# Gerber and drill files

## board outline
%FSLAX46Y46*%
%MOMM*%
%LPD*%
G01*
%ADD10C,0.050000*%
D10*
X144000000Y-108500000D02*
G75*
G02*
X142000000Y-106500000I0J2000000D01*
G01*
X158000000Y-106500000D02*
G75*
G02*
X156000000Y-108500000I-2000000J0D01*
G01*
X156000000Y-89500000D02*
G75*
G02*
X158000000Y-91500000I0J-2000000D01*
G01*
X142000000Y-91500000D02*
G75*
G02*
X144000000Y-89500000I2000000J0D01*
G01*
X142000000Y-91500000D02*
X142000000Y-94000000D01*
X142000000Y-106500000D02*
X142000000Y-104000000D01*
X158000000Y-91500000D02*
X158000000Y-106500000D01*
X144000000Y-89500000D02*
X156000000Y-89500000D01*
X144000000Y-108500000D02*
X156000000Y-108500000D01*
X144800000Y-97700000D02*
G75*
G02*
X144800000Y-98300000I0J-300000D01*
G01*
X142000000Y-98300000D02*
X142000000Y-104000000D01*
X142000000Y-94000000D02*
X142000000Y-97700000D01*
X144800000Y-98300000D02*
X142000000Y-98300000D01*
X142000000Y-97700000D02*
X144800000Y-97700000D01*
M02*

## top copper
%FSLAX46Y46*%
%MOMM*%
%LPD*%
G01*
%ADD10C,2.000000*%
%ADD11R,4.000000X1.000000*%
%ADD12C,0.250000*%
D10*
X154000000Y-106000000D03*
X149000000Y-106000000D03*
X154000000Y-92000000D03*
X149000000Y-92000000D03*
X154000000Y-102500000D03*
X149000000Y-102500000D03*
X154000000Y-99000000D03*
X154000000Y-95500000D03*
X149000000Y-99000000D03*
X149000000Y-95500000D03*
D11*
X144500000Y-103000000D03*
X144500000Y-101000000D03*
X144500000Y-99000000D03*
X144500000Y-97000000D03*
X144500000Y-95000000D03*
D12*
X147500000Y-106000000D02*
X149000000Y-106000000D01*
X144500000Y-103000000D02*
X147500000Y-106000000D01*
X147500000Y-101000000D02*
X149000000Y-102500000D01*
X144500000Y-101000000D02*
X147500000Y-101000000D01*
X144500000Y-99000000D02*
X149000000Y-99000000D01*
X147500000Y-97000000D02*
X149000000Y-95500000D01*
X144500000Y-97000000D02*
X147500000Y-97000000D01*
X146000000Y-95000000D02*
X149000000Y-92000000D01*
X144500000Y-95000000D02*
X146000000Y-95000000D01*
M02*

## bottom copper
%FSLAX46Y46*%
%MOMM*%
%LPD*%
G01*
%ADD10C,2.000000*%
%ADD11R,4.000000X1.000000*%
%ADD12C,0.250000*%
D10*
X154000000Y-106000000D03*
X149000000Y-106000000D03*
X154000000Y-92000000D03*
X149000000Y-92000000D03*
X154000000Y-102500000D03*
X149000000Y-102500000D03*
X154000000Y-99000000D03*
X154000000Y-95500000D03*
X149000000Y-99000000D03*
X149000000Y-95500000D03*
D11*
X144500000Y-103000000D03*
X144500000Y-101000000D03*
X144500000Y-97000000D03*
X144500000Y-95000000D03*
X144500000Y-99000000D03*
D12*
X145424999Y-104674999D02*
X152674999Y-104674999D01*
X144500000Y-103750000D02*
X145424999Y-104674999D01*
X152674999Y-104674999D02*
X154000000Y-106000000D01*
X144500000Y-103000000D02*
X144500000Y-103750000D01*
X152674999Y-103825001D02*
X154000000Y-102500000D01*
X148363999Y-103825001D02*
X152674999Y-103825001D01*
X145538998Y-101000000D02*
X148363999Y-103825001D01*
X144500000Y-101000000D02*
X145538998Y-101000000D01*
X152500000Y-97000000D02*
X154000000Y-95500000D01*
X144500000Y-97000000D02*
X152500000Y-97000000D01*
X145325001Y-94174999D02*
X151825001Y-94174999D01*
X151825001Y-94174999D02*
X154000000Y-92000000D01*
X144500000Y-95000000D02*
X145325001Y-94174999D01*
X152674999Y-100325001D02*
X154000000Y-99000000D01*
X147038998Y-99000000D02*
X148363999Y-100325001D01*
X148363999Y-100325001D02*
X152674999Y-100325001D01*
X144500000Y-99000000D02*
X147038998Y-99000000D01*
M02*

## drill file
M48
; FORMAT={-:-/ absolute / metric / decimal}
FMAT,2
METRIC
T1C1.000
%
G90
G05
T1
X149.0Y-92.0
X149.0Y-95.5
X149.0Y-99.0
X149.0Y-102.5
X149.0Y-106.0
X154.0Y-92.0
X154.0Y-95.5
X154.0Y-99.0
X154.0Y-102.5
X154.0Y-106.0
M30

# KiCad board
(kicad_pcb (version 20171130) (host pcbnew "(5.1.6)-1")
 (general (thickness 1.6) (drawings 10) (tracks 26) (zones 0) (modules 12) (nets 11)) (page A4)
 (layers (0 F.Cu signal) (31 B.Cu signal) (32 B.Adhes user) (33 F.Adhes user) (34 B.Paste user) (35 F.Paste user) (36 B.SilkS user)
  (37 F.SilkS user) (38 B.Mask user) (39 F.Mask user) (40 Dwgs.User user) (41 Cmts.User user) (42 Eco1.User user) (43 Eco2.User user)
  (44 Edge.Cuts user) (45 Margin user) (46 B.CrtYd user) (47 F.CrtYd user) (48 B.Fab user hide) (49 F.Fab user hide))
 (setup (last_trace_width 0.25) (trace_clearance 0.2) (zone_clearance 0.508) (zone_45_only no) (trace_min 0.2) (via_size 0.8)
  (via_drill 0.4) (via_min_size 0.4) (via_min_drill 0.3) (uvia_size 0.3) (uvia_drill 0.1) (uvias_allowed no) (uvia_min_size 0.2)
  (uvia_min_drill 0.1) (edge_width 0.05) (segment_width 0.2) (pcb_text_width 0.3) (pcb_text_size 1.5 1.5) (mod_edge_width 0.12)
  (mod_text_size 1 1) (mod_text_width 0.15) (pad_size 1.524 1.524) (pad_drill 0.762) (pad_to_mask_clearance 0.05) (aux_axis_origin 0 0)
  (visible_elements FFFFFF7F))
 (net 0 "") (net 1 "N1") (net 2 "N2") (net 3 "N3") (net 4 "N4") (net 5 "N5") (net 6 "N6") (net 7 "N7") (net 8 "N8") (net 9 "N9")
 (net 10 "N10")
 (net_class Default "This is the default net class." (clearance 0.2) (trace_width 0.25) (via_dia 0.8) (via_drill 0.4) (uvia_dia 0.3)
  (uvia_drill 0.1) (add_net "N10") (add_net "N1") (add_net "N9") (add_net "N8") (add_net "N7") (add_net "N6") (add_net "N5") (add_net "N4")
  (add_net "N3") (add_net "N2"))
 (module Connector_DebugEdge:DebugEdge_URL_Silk (layer B.Cu) (at 151.5 98.5 270)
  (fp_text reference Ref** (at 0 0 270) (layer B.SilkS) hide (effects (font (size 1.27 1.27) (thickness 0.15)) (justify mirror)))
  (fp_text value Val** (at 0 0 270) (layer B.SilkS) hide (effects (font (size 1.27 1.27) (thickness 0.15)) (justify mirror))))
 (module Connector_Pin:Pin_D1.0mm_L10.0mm (layer F.Cu) (at 154 106 90)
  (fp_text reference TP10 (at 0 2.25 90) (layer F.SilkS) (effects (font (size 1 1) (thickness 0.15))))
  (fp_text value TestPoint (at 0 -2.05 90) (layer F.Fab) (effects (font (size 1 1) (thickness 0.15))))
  (pad 1 thru_hole circle (at 0 0 90) (size 2 2) (drill 1) (layers *.Cu *.Mask) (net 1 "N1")))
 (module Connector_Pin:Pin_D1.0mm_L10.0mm (layer F.Cu) (at 149 106 90)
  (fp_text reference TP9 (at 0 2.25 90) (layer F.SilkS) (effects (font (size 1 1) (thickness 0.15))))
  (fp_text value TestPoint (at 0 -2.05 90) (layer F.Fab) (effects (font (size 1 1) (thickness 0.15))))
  (pad 1 thru_hole circle (at 0 0 90) (size 2 2) (drill 1) (layers *.Cu *.Mask) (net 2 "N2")))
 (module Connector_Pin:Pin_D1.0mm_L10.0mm (layer F.Cu) (at 154 92 90)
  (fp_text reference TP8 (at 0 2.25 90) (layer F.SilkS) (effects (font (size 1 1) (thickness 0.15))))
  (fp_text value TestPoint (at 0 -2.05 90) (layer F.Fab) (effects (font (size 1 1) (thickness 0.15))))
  (pad 1 thru_hole circle (at 0 0 90) (size 2 2) (drill 1) (layers *.Cu *.Mask) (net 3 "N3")))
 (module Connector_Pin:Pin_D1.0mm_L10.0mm (layer F.Cu) (at 149 92 90)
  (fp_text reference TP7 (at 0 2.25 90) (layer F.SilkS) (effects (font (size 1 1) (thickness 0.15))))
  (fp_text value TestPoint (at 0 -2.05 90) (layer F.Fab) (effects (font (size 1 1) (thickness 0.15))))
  (pad 1 thru_hole circle (at 0 0 90) (size 2 2) (drill 1) (layers *.Cu *.Mask) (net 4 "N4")))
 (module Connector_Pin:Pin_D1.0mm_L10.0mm (layer F.Cu) (at 154 102.5 90)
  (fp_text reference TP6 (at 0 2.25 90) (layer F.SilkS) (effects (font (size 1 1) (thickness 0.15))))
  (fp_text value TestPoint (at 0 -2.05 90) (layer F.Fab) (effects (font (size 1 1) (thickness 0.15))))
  (pad 1 thru_hole circle (at 0 0 90) (size 2 2) (drill 1) (layers *.Cu *.Mask) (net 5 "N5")))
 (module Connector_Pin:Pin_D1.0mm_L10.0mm (layer F.Cu) (at 149 102.5 90)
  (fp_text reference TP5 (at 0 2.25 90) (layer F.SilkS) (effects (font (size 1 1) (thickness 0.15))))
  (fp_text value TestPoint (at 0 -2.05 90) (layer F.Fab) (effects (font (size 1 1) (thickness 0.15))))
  (pad 1 thru_hole circle (at 0 0 90) (size 2 2) (drill 1) (layers *.Cu *.Mask) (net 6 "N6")))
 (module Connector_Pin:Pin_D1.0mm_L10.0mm (layer F.Cu) (at 154 99 90)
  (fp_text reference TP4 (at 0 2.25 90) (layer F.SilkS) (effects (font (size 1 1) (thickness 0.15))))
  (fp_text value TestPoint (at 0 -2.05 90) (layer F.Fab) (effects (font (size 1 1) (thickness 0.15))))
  (pad 1 thru_hole circle (at 0 0 90) (size 2 2) (drill 1) (layers *.Cu *.Mask) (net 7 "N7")))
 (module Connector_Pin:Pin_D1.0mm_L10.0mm (layer F.Cu) (at 154 95.5 90)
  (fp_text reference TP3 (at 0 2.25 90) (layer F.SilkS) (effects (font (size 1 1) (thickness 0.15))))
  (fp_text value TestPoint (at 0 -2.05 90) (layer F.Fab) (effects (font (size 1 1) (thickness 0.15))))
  (pad 1 thru_hole circle (at 0 0 90) (size 2 2) (drill 1) (layers *.Cu *.Mask) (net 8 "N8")))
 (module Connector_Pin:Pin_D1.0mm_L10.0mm (layer F.Cu) (at 149 99 90)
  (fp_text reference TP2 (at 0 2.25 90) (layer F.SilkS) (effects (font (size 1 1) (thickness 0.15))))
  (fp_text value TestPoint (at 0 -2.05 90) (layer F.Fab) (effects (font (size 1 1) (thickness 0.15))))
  (pad 1 thru_hole circle (at 0 0 90) (size 2 2) (drill 1) (layers *.Cu *.Mask) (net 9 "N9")))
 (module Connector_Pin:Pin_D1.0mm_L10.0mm (layer F.Cu) (at 149 95.5 90)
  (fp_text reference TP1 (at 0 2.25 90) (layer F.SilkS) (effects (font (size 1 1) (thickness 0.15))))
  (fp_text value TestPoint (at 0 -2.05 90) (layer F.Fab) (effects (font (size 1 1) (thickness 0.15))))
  (pad 1 thru_hole circle (at 0 0 90) (size 2 2) (drill 1) (layers *.Cu *.Mask) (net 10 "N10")))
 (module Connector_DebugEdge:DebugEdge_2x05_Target (layer F.Cu) (at 142 99 270)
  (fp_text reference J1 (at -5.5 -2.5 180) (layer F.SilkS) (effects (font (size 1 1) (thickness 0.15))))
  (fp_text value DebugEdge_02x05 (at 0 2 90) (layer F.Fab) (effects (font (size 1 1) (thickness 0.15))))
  (fp_arc (start -1 -2.8) (end -1.3 -2.8) (angle 180) (layer Edge.Cuts) (width 0.05))
  (fp_line (start -0.7 0) (end 5 0) (layer Edge.Cuts) (width 0.05))
  (fp_line (start -5 0) (end -1.3 0) (layer Edge.Cuts) (width 0.05))
  (fp_line (start -0.7 -2.8) (end -0.7 0) (layer Edge.Cuts) (width 0.05))
  (fp_line (start -1.3 0) (end -1.3 -2.8) (layer Edge.Cuts) (width 0.05))
  (pad 9 smd rect (at 4 -2.5 90) (size 1 4) (layers F.Cu F.Mask) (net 2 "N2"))
  (pad 5 smd rect (at 2 -2.5 90) (size 1 4) (layers F.Cu F.Mask) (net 6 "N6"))
  (pad 2 smd rect (at 0 -2.5 90) (size 1 4) (layers F.Cu F.Mask) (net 9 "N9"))
  (pad 1 smd rect (at -2 -2.5 90) (size 1 4) (layers F.Cu F.Mask) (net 10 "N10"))
  (pad 7 smd rect (at -4 -2.5 90) (size 1 4) (layers F.Cu F.Mask) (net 4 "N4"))
  (pad 10 smd rect (at 4 -2.5 90) (size 1 4) (layers B.Cu B.Mask) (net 1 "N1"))
  (pad 6 smd rect (at 2 -2.5 90) (size 1 4) (layers B.Cu B.Mask) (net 5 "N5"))
  (pad 3 smd rect (at -2 -2.5 90) (size 1 4) (layers B.Cu B.Mask) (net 8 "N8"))
  (pad 8 smd rect (at -4 -2.5 90) (size 1 4) (layers B.Cu B.Mask) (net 3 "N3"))
  (pad 4 smd rect (at 0 -2.5 90) (size 1 4) (layers B.Cu B.Mask) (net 7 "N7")))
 (gr_arc (start 144 106.5) (end 142 106.5) (angle -90) (layer Edge.Cuts) (width 0.05))
 (gr_arc (start 156 106.5) (end 156 108.5) (angle -90) (layer Edge.Cuts) (width 0.05))
 (gr_arc (start 156 91.5) (end 158 91.5) (angle -90) (layer Edge.Cuts) (width 0.05))
 (gr_arc (start 144 91.5) (end 144 89.5) (angle -90) (layer Edge.Cuts) (width 0.05))
 (gr_line (start 142 91.5) (end 142 94) (layer Edge.Cuts) (width 0.05))
 (gr_line (start 142 106.5) (end 142 104) (layer Edge.Cuts) (width 0.05))
 (gr_line (start 158 91.5) (end 158 106.5) (layer Edge.Cuts) (width 0.05))
 (gr_line (start 144 89.5) (end 156 89.5) (layer Edge.Cuts) (width 0.05))
 (gr_line (start 144 108.5) (end 156 108.5) (layer Edge.Cuts) (width 0.05))
 (segment (start 147.5 106) (end 149 106) (width 0.25) (layer F.Cu) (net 2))
 (segment (start 144.5 103) (end 147.5 106) (width 0.25) (layer F.Cu) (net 2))
 (segment (start 147.5 101) (end 149 102.5) (width 0.25) (layer F.Cu) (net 6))
 (segment (start 144.5 101) (end 147.5 101) (width 0.25) (layer F.Cu) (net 6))
 (segment (start 144.5 99) (end 149 99) (width 0.25) (layer F.Cu) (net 9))
 (segment (start 147.5 97) (end 149 95.5) (width 0.25) (layer F.Cu) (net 10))
 (segment (start 144.5 97) (end 147.5 97) (width 0.25) (layer F.Cu) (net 10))
 (segment (start 146 95) (end 149 92) (width 0.25) (layer F.Cu) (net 4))
 (segment (start 144.5 95) (end 146 95) (width 0.25) (layer F.Cu) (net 4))
 (segment (start 145.424999 104.674999) (end 152.674999 104.674999) (width 0.25) (layer B.Cu) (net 1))
 (segment (start 144.5 103.75) (end 145.424999 104.674999) (width 0.25) (layer B.Cu) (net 1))
 (segment (start 152.674999 104.674999) (end 154 106) (width 0.25) (layer B.Cu) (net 1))
 (segment (start 144.5 103) (end 144.5 103.75) (width 0.25) (layer B.Cu) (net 1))
 (segment (start 152.674999 103.825001) (end 154 102.5) (width 0.25) (layer B.Cu) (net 5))
 (segment (start 148.363999 103.825001) (end 152.674999 103.825001) (width 0.25) (layer B.Cu) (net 5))
 (segment (start 145.538998 101) (end 148.363999 103.825001) (width 0.25) (layer B.Cu) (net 5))
 (segment (start 144.5 101) (end 145.538998 101) (width 0.25) (layer B.Cu) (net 5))
 (segment (start 152.5 97) (end 154 95.5) (width 0.25) (layer B.Cu) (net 8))
 (segment (start 144.5 97) (end 152.5 97) (width 0.25) (layer B.Cu) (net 8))
 (segment (start 145.325001 94.174999) (end 151.825001 94.174999) (width 0.25) (layer B.Cu) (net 3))
 (segment (start 151.825001 94.174999) (end 154 92) (width 0.25) (layer B.Cu) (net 3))
 (segment (start 144.5 95) (end 145.325001 94.174999) (width 0.25) (layer B.Cu) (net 3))
 (segment (start 152.674999 100.325001) (end 154 99) (width 0.25) (layer B.Cu) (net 7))
 (segment (start 147.038998 99) (end 148.363999 100.325001) (width 0.25) (layer B.Cu) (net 7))
 (segment (start 148.363999 100.325001) (end 152.674999 100.325001) (width 0.25) (layer B.Cu) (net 7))
 (segment (start 144.5 99) (end 147.038998 99) (width 0.25) (layer B.Cu) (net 7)))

